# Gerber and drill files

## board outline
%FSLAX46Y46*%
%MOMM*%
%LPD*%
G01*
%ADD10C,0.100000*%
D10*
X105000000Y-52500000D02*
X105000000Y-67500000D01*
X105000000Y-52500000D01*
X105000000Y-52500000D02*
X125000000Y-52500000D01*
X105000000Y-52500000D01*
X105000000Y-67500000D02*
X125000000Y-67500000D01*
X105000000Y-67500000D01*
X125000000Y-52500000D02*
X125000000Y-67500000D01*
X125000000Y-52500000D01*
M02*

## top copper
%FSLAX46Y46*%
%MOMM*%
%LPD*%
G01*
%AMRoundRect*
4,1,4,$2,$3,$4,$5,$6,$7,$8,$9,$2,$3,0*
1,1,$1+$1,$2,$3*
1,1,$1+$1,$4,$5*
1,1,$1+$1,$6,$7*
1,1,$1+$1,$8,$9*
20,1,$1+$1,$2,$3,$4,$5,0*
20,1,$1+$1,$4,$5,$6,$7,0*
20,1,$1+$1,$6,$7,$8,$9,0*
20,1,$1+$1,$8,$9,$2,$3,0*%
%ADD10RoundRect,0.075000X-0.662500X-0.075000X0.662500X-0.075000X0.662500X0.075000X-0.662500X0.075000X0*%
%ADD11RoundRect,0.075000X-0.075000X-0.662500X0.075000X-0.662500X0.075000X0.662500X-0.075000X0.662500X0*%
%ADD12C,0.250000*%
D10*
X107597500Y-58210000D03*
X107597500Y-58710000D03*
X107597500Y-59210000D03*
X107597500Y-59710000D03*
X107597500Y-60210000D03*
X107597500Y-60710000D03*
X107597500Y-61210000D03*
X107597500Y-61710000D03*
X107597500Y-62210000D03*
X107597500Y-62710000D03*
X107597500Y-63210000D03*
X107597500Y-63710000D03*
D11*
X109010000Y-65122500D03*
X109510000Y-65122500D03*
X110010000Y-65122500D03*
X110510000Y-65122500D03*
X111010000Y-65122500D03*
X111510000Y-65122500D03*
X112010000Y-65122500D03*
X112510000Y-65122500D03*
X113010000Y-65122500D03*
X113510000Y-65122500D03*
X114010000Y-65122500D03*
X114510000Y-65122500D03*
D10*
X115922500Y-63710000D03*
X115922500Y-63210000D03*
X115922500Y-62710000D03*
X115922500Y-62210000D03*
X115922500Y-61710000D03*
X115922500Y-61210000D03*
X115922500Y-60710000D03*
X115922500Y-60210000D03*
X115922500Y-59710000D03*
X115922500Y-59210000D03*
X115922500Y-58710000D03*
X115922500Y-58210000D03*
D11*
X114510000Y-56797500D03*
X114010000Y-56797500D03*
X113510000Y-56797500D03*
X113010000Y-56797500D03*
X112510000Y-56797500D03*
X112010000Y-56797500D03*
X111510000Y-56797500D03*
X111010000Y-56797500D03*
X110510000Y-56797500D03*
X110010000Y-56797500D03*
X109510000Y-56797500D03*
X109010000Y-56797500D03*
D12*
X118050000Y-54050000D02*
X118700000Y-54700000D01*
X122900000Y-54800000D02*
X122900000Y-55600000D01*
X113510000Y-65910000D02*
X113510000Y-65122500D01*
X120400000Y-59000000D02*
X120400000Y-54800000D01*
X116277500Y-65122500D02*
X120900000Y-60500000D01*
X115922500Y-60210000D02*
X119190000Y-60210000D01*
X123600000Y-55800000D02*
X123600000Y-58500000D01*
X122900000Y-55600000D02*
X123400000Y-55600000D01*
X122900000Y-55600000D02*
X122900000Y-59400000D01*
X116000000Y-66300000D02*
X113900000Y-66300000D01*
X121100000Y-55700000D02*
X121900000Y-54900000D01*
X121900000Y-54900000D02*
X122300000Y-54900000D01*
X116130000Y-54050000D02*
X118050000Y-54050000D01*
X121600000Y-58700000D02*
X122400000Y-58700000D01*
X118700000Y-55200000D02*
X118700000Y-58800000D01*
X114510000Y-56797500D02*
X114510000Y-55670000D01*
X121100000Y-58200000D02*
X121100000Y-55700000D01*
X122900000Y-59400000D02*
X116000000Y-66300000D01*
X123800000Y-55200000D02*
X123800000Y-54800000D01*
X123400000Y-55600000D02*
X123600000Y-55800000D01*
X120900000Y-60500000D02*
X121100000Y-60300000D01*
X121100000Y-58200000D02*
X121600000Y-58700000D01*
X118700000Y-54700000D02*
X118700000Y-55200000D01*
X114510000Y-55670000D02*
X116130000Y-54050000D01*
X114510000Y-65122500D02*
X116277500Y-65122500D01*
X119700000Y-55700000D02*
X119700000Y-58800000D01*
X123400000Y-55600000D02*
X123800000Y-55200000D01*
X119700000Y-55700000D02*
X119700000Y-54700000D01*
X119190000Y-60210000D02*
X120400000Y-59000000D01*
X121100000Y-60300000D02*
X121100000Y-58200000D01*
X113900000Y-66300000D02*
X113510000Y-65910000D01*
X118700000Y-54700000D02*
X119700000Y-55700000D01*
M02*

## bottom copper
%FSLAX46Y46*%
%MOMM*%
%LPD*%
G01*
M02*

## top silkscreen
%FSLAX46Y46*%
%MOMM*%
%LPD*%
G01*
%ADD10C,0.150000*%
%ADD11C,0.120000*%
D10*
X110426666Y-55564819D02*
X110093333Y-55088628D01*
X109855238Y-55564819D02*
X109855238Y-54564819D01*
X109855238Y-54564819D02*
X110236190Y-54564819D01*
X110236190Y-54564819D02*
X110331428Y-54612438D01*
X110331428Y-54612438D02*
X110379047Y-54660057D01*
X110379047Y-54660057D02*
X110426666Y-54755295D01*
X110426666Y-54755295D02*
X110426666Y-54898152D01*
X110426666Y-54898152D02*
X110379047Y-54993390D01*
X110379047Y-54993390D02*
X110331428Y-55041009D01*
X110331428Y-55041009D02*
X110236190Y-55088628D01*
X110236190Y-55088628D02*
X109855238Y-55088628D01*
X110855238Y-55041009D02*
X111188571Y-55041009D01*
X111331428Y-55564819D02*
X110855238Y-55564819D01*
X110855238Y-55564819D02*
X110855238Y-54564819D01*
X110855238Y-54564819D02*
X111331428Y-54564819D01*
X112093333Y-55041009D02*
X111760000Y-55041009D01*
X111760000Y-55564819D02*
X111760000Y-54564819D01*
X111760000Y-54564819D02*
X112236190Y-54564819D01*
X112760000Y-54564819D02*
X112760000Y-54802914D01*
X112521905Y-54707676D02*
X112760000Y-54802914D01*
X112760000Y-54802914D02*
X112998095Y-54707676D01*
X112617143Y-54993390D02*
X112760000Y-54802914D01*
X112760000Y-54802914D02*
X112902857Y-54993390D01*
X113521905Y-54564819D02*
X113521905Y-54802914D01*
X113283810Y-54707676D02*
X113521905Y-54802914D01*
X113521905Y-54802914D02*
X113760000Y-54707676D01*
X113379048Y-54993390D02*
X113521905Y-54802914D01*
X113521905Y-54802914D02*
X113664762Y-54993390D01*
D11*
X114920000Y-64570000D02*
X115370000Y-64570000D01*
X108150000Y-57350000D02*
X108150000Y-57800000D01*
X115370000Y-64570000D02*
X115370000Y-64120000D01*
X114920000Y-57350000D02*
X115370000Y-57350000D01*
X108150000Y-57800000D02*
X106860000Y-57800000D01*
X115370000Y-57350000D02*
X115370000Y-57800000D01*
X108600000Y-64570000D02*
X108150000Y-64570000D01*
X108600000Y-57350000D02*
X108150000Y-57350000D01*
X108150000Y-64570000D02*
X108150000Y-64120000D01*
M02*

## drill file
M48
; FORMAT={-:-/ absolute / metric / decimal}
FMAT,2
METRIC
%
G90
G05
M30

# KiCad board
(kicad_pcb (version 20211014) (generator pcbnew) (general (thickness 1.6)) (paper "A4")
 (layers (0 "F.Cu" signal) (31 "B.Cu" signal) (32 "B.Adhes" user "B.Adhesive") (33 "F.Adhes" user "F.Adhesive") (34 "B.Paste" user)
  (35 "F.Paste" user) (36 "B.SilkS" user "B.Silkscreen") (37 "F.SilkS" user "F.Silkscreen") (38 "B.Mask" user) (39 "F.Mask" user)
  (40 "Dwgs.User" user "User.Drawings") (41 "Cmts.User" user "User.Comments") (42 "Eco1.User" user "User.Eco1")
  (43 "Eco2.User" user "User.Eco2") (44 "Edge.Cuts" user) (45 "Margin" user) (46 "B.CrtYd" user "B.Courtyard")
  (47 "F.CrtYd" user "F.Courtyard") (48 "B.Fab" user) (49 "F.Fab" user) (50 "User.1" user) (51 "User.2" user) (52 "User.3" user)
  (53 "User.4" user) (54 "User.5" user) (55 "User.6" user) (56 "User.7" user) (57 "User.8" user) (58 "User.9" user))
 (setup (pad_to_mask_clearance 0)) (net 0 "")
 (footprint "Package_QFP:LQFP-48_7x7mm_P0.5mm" (layer "F.Cu") (at 111.76 60.96)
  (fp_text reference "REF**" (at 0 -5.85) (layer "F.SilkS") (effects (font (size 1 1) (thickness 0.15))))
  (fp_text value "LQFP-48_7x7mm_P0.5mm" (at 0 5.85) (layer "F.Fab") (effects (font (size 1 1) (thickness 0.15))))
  (fp_line (start 3.16 3.61) (end 3.61 3.61) (layer "F.SilkS") (width 0.12))
  (fp_line (start -3.61 -3.61) (end -3.61 -3.16) (layer "F.SilkS") (width 0.12))
  (fp_line (start 3.61 3.61) (end 3.61 3.16) (layer "F.SilkS") (width 0.12))
  (fp_line (start 3.16 -3.61) (end 3.61 -3.61) (layer "F.SilkS") (width 0.12))
  (fp_line (start -3.61 -3.16) (end -4.9 -3.16) (layer "F.SilkS") (width 0.12))
  (fp_line (start 3.61 -3.61) (end 3.61 -3.16) (layer "F.SilkS") (width 0.12))
  (fp_line (start -3.16 3.61) (end -3.61 3.61) (layer "F.SilkS") (width 0.12))
  (fp_line (start -3.16 -3.61) (end -3.61 -3.61) (layer "F.SilkS") (width 0.12))
  (fp_line (start -3.61 3.61) (end -3.61 3.16) (layer "F.SilkS") (width 0.12))
  (pad "1" smd roundrect (at -4.1625 -2.75) (size 1.475 0.3) (layers "F.Cu" "F.Paste" "F.Mask") (roundrect_rratio 0.25))
  (pad "2" smd roundrect (at -4.1625 -2.25) (size 1.475 0.3) (layers "F.Cu" "F.Paste" "F.Mask") (roundrect_rratio 0.25))
  (pad "3" smd roundrect (at -4.1625 -1.75) (size 1.475 0.3) (layers "F.Cu" "F.Paste" "F.Mask") (roundrect_rratio 0.25))
  (pad "4" smd roundrect (at -4.1625 -1.25) (size 1.475 0.3) (layers "F.Cu" "F.Paste" "F.Mask") (roundrect_rratio 0.25))
  (pad "5" smd roundrect (at -4.1625 -0.75) (size 1.475 0.3) (layers "F.Cu" "F.Paste" "F.Mask") (roundrect_rratio 0.25))
  (pad "6" smd roundrect (at -4.1625 -0.25) (size 1.475 0.3) (layers "F.Cu" "F.Paste" "F.Mask") (roundrect_rratio 0.25))
  (pad "7" smd roundrect (at -4.1625 0.25) (size 1.475 0.3) (layers "F.Cu" "F.Paste" "F.Mask") (roundrect_rratio 0.25))
  (pad "8" smd roundrect (at -4.1625 0.75) (size 1.475 0.3) (layers "F.Cu" "F.Paste" "F.Mask") (roundrect_rratio 0.25))
  (pad "9" smd roundrect (at -4.1625 1.25) (size 1.475 0.3) (layers "F.Cu" "F.Paste" "F.Mask") (roundrect_rratio 0.25))
  (pad "10" smd roundrect (at -4.1625 1.75) (size 1.475 0.3) (layers "F.Cu" "F.Paste" "F.Mask") (roundrect_rratio 0.25))
  (pad "11" smd roundrect (at -4.1625 2.25) (size 1.475 0.3) (layers "F.Cu" "F.Paste" "F.Mask") (roundrect_rratio 0.25))
  (pad "12" smd roundrect (at -4.1625 2.75) (size 1.475 0.3) (layers "F.Cu" "F.Paste" "F.Mask") (roundrect_rratio 0.25))
  (pad "13" smd roundrect (at -2.75 4.1625) (size 0.3 1.475) (layers "F.Cu" "F.Paste" "F.Mask") (roundrect_rratio 0.25))
  (pad "14" smd roundrect (at -2.25 4.1625) (size 0.3 1.475) (layers "F.Cu" "F.Paste" "F.Mask") (roundrect_rratio 0.25))
  (pad "15" smd roundrect (at -1.75 4.1625) (size 0.3 1.475) (layers "F.Cu" "F.Paste" "F.Mask") (roundrect_rratio 0.25))
  (pad "16" smd roundrect (at -1.25 4.1625) (size 0.3 1.475) (layers "F.Cu" "F.Paste" "F.Mask") (roundrect_rratio 0.25))
  (pad "17" smd roundrect (at -0.75 4.1625) (size 0.3 1.475) (layers "F.Cu" "F.Paste" "F.Mask") (roundrect_rratio 0.25))
  (pad "18" smd roundrect (at -0.25 4.1625) (size 0.3 1.475) (layers "F.Cu" "F.Paste" "F.Mask") (roundrect_rratio 0.25))
  (pad "19" smd roundrect (at 0.25 4.1625) (size 0.3 1.475) (layers "F.Cu" "F.Paste" "F.Mask") (roundrect_rratio 0.25))
  (pad "20" smd roundrect (at 0.75 4.1625) (size 0.3 1.475) (layers "F.Cu" "F.Paste" "F.Mask") (roundrect_rratio 0.25))
  (pad "21" smd roundrect (at 1.25 4.1625) (size 0.3 1.475) (layers "F.Cu" "F.Paste" "F.Mask") (roundrect_rratio 0.25))
  (pad "22" smd roundrect (at 1.75 4.1625) (size 0.3 1.475) (layers "F.Cu" "F.Paste" "F.Mask") (roundrect_rratio 0.25))
  (pad "23" smd roundrect (at 2.25 4.1625) (size 0.3 1.475) (layers "F.Cu" "F.Paste" "F.Mask") (roundrect_rratio 0.25))
  (pad "24" smd roundrect (at 2.75 4.1625) (size 0.3 1.475) (layers "F.Cu" "F.Paste" "F.Mask") (roundrect_rratio 0.25))
  (pad "25" smd roundrect (at 4.1625 2.75) (size 1.475 0.3) (layers "F.Cu" "F.Paste" "F.Mask") (roundrect_rratio 0.25))
  (pad "26" smd roundrect (at 4.1625 2.25) (size 1.475 0.3) (layers "F.Cu" "F.Paste" "F.Mask") (roundrect_rratio 0.25))
  (pad "27" smd roundrect (at 4.1625 1.75) (size 1.475 0.3) (layers "F.Cu" "F.Paste" "F.Mask") (roundrect_rratio 0.25))
  (pad "28" smd roundrect (at 4.1625 1.25) (size 1.475 0.3) (layers "F.Cu" "F.Paste" "F.Mask") (roundrect_rratio 0.25))
  (pad "29" smd roundrect (at 4.1625 0.75) (size 1.475 0.3) (layers "F.Cu" "F.Paste" "F.Mask") (roundrect_rratio 0.25))
  (pad "30" smd roundrect (at 4.1625 0.25) (size 1.475 0.3) (layers "F.Cu" "F.Paste" "F.Mask") (roundrect_rratio 0.25))
  (pad "31" smd roundrect (at 4.1625 -0.25) (size 1.475 0.3) (layers "F.Cu" "F.Paste" "F.Mask") (roundrect_rratio 0.25))
  (pad "32" smd roundrect (at 4.1625 -0.75) (size 1.475 0.3) (layers "F.Cu" "F.Paste" "F.Mask") (roundrect_rratio 0.25))
  (pad "33" smd roundrect (at 4.1625 -1.25) (size 1.475 0.3) (layers "F.Cu" "F.Paste" "F.Mask") (roundrect_rratio 0.25))
  (pad "34" smd roundrect (at 4.1625 -1.75) (size 1.475 0.3) (layers "F.Cu" "F.Paste" "F.Mask") (roundrect_rratio 0.25))
  (pad "35" smd roundrect (at 4.1625 -2.25) (size 1.475 0.3) (layers "F.Cu" "F.Paste" "F.Mask") (roundrect_rratio 0.25))
  (pad "36" smd roundrect (at 4.1625 -2.75) (size 1.475 0.3) (layers "F.Cu" "F.Paste" "F.Mask") (roundrect_rratio 0.25))
  (pad "37" smd roundrect (at 2.75 -4.1625) (size 0.3 1.475) (layers "F.Cu" "F.Paste" "F.Mask") (roundrect_rratio 0.25))
  (pad "38" smd roundrect (at 2.25 -4.1625) (size 0.3 1.475) (layers "F.Cu" "F.Paste" "F.Mask") (roundrect_rratio 0.25))
  (pad "39" smd roundrect (at 1.75 -4.1625) (size 0.3 1.475) (layers "F.Cu" "F.Paste" "F.Mask") (roundrect_rratio 0.25))
  (pad "40" smd roundrect (at 1.25 -4.1625) (size 0.3 1.475) (layers "F.Cu" "F.Paste" "F.Mask") (roundrect_rratio 0.25))
  (pad "41" smd roundrect (at 0.75 -4.1625) (size 0.3 1.475) (layers "F.Cu" "F.Paste" "F.Mask") (roundrect_rratio 0.25))
  (pad "42" smd roundrect (at 0.25 -4.1625) (size 0.3 1.475) (layers "F.Cu" "F.Paste" "F.Mask") (roundrect_rratio 0.25))
  (pad "43" smd roundrect (at -0.25 -4.1625) (size 0.3 1.475) (layers "F.Cu" "F.Paste" "F.Mask") (roundrect_rratio 0.25))
  (pad "44" smd roundrect (at -0.75 -4.1625) (size 0.3 1.475) (layers "F.Cu" "F.Paste" "F.Mask") (roundrect_rratio 0.25))
  (pad "45" smd roundrect (at -1.25 -4.1625) (size 0.3 1.475) (layers "F.Cu" "F.Paste" "F.Mask") (roundrect_rratio 0.25))
  (pad "46" smd roundrect (at -1.75 -4.1625) (size 0.3 1.475) (layers "F.Cu" "F.Paste" "F.Mask") (roundrect_rratio 0.25))
  (pad "47" smd roundrect (at -2.25 -4.1625) (size 0.3 1.475) (layers "F.Cu" "F.Paste" "F.Mask") (roundrect_rratio 0.25))
  (pad "48" smd roundrect (at -2.75 -4.1625) (size 0.3 1.475) (layers "F.Cu" "F.Paste" "F.Mask") (roundrect_rratio 0.25)))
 (gr_rect (start 105 67.5) (end 105 52.5) (layer "Edge.Cuts") (width 0.1) (fill none))
 (gr_rect (start 125 52.5) (end 105 52.5) (layer "Edge.Cuts") (width 0.1) (fill none))
 (gr_rect (start 105 67.5) (end 125 67.5) (layer "Edge.Cuts") (width 0.1) (fill none))
 (gr_rect (start 125 52.5) (end 125 67.5) (layer "Edge.Cuts") (width 0.1) (fill none))
 (segment (start 118.05 54.05) (end 118.7 54.7) (width 0.25) (layer "F.Cu") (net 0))
 (segment (start 122.9 54.8) (end 122.9 55.6) (width 0.25) (layer "F.Cu") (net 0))
 (segment (start 113.51 65.91) (end 113.51 65.1225) (width 0.25) (layer "F.Cu") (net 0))
 (segment (start 120.4 59) (end 120.4 54.8) (width 0.25) (layer "F.Cu") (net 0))
 (segment (start 116.2775 65.1225) (end 120.9 60.5) (width 0.25) (layer "F.Cu") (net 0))
 (segment (start 115.9225 60.21) (end 119.19 60.21) (width 0.25) (layer "F.Cu") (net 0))
 (segment (start 123.6 55.8) (end 123.6 58.5) (width 0.25) (layer "F.Cu") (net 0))
 (segment (start 122.9 55.6) (end 123.4 55.6) (width 0.25) (layer "F.Cu") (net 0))
 (segment (start 122.9 55.6) (end 122.9 59.4) (width 0.25) (layer "F.Cu") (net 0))
 (segment (start 116 66.3) (end 113.9 66.3) (width 0.25) (layer "F.Cu") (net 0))
 (segment (start 121.1 55.7) (end 121.9 54.9) (width 0.25) (layer "F.Cu") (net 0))
 (segment (start 121.9 54.9) (end 122.3 54.9) (width 0.25) (layer "F.Cu") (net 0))
 (segment (start 116.13 54.05) (end 118.05 54.05) (width 0.25) (layer "F.Cu") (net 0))
 (segment (start 121.6 58.7) (end 122.4 58.7) (width 0.25) (layer "F.Cu") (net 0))
 (segment (start 118.7 55.2) (end 118.7 58.8) (width 0.25) (layer "F.Cu") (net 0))
 (segment (start 114.51 56.7975) (end 114.51 55.67) (width 0.25) (layer "F.Cu") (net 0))
 (segment (start 121.1 58.2) (end 121.1 55.7) (width 0.25) (layer "F.Cu") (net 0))
 (segment (start 122.9 59.4) (end 116 66.3) (width 0.25) (layer "F.Cu") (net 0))
 (segment (start 123.8 55.2) (end 123.8 54.8) (width 0.25) (layer "F.Cu") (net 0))
 (segment (start 123.4 55.6) (end 123.6 55.8) (width 0.25) (layer "F.Cu") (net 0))
 (segment (start 120.9 60.5) (end 121.1 60.3) (width 0.25) (layer "F.Cu") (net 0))
 (segment (start 121.1 58.2) (end 121.6 58.7) (width 0.25) (layer "F.Cu") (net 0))
 (segment (start 118.7 54.7) (end 118.7 55.2) (width 0.25) (layer "F.Cu") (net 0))
 (segment (start 114.51 55.67) (end 116.13 54.05) (width 0.25) (layer "F.Cu") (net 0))
 (segment (start 114.51 65.1225) (end 116.2775 65.1225) (width 0.25) (layer "F.Cu") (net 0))
 (segment (start 119.7 55.7) (end 119.7 58.8) (width 0.25) (layer "F.Cu") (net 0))
 (segment (start 123.4 55.6) (end 123.8 55.2) (width 0.25) (layer "F.Cu") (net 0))
 (segment (start 119.7 55.7) (end 119.7 54.7) (width 0.25) (layer "F.Cu") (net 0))
 (segment (start 119.19 60.21) (end 120.4 59) (width 0.25) (layer "F.Cu") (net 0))
 (segment (start 121.1 60.3) (end 121.1 58.2) (width 0.25) (layer "F.Cu") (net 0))
 (segment (start 113.9 66.3) (end 113.51 65.91) (width 0.25) (layer "F.Cu") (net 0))
 (segment (start 118.7 54.7) (end 119.7 55.7) (width 0.25) (layer "F.Cu") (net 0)))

